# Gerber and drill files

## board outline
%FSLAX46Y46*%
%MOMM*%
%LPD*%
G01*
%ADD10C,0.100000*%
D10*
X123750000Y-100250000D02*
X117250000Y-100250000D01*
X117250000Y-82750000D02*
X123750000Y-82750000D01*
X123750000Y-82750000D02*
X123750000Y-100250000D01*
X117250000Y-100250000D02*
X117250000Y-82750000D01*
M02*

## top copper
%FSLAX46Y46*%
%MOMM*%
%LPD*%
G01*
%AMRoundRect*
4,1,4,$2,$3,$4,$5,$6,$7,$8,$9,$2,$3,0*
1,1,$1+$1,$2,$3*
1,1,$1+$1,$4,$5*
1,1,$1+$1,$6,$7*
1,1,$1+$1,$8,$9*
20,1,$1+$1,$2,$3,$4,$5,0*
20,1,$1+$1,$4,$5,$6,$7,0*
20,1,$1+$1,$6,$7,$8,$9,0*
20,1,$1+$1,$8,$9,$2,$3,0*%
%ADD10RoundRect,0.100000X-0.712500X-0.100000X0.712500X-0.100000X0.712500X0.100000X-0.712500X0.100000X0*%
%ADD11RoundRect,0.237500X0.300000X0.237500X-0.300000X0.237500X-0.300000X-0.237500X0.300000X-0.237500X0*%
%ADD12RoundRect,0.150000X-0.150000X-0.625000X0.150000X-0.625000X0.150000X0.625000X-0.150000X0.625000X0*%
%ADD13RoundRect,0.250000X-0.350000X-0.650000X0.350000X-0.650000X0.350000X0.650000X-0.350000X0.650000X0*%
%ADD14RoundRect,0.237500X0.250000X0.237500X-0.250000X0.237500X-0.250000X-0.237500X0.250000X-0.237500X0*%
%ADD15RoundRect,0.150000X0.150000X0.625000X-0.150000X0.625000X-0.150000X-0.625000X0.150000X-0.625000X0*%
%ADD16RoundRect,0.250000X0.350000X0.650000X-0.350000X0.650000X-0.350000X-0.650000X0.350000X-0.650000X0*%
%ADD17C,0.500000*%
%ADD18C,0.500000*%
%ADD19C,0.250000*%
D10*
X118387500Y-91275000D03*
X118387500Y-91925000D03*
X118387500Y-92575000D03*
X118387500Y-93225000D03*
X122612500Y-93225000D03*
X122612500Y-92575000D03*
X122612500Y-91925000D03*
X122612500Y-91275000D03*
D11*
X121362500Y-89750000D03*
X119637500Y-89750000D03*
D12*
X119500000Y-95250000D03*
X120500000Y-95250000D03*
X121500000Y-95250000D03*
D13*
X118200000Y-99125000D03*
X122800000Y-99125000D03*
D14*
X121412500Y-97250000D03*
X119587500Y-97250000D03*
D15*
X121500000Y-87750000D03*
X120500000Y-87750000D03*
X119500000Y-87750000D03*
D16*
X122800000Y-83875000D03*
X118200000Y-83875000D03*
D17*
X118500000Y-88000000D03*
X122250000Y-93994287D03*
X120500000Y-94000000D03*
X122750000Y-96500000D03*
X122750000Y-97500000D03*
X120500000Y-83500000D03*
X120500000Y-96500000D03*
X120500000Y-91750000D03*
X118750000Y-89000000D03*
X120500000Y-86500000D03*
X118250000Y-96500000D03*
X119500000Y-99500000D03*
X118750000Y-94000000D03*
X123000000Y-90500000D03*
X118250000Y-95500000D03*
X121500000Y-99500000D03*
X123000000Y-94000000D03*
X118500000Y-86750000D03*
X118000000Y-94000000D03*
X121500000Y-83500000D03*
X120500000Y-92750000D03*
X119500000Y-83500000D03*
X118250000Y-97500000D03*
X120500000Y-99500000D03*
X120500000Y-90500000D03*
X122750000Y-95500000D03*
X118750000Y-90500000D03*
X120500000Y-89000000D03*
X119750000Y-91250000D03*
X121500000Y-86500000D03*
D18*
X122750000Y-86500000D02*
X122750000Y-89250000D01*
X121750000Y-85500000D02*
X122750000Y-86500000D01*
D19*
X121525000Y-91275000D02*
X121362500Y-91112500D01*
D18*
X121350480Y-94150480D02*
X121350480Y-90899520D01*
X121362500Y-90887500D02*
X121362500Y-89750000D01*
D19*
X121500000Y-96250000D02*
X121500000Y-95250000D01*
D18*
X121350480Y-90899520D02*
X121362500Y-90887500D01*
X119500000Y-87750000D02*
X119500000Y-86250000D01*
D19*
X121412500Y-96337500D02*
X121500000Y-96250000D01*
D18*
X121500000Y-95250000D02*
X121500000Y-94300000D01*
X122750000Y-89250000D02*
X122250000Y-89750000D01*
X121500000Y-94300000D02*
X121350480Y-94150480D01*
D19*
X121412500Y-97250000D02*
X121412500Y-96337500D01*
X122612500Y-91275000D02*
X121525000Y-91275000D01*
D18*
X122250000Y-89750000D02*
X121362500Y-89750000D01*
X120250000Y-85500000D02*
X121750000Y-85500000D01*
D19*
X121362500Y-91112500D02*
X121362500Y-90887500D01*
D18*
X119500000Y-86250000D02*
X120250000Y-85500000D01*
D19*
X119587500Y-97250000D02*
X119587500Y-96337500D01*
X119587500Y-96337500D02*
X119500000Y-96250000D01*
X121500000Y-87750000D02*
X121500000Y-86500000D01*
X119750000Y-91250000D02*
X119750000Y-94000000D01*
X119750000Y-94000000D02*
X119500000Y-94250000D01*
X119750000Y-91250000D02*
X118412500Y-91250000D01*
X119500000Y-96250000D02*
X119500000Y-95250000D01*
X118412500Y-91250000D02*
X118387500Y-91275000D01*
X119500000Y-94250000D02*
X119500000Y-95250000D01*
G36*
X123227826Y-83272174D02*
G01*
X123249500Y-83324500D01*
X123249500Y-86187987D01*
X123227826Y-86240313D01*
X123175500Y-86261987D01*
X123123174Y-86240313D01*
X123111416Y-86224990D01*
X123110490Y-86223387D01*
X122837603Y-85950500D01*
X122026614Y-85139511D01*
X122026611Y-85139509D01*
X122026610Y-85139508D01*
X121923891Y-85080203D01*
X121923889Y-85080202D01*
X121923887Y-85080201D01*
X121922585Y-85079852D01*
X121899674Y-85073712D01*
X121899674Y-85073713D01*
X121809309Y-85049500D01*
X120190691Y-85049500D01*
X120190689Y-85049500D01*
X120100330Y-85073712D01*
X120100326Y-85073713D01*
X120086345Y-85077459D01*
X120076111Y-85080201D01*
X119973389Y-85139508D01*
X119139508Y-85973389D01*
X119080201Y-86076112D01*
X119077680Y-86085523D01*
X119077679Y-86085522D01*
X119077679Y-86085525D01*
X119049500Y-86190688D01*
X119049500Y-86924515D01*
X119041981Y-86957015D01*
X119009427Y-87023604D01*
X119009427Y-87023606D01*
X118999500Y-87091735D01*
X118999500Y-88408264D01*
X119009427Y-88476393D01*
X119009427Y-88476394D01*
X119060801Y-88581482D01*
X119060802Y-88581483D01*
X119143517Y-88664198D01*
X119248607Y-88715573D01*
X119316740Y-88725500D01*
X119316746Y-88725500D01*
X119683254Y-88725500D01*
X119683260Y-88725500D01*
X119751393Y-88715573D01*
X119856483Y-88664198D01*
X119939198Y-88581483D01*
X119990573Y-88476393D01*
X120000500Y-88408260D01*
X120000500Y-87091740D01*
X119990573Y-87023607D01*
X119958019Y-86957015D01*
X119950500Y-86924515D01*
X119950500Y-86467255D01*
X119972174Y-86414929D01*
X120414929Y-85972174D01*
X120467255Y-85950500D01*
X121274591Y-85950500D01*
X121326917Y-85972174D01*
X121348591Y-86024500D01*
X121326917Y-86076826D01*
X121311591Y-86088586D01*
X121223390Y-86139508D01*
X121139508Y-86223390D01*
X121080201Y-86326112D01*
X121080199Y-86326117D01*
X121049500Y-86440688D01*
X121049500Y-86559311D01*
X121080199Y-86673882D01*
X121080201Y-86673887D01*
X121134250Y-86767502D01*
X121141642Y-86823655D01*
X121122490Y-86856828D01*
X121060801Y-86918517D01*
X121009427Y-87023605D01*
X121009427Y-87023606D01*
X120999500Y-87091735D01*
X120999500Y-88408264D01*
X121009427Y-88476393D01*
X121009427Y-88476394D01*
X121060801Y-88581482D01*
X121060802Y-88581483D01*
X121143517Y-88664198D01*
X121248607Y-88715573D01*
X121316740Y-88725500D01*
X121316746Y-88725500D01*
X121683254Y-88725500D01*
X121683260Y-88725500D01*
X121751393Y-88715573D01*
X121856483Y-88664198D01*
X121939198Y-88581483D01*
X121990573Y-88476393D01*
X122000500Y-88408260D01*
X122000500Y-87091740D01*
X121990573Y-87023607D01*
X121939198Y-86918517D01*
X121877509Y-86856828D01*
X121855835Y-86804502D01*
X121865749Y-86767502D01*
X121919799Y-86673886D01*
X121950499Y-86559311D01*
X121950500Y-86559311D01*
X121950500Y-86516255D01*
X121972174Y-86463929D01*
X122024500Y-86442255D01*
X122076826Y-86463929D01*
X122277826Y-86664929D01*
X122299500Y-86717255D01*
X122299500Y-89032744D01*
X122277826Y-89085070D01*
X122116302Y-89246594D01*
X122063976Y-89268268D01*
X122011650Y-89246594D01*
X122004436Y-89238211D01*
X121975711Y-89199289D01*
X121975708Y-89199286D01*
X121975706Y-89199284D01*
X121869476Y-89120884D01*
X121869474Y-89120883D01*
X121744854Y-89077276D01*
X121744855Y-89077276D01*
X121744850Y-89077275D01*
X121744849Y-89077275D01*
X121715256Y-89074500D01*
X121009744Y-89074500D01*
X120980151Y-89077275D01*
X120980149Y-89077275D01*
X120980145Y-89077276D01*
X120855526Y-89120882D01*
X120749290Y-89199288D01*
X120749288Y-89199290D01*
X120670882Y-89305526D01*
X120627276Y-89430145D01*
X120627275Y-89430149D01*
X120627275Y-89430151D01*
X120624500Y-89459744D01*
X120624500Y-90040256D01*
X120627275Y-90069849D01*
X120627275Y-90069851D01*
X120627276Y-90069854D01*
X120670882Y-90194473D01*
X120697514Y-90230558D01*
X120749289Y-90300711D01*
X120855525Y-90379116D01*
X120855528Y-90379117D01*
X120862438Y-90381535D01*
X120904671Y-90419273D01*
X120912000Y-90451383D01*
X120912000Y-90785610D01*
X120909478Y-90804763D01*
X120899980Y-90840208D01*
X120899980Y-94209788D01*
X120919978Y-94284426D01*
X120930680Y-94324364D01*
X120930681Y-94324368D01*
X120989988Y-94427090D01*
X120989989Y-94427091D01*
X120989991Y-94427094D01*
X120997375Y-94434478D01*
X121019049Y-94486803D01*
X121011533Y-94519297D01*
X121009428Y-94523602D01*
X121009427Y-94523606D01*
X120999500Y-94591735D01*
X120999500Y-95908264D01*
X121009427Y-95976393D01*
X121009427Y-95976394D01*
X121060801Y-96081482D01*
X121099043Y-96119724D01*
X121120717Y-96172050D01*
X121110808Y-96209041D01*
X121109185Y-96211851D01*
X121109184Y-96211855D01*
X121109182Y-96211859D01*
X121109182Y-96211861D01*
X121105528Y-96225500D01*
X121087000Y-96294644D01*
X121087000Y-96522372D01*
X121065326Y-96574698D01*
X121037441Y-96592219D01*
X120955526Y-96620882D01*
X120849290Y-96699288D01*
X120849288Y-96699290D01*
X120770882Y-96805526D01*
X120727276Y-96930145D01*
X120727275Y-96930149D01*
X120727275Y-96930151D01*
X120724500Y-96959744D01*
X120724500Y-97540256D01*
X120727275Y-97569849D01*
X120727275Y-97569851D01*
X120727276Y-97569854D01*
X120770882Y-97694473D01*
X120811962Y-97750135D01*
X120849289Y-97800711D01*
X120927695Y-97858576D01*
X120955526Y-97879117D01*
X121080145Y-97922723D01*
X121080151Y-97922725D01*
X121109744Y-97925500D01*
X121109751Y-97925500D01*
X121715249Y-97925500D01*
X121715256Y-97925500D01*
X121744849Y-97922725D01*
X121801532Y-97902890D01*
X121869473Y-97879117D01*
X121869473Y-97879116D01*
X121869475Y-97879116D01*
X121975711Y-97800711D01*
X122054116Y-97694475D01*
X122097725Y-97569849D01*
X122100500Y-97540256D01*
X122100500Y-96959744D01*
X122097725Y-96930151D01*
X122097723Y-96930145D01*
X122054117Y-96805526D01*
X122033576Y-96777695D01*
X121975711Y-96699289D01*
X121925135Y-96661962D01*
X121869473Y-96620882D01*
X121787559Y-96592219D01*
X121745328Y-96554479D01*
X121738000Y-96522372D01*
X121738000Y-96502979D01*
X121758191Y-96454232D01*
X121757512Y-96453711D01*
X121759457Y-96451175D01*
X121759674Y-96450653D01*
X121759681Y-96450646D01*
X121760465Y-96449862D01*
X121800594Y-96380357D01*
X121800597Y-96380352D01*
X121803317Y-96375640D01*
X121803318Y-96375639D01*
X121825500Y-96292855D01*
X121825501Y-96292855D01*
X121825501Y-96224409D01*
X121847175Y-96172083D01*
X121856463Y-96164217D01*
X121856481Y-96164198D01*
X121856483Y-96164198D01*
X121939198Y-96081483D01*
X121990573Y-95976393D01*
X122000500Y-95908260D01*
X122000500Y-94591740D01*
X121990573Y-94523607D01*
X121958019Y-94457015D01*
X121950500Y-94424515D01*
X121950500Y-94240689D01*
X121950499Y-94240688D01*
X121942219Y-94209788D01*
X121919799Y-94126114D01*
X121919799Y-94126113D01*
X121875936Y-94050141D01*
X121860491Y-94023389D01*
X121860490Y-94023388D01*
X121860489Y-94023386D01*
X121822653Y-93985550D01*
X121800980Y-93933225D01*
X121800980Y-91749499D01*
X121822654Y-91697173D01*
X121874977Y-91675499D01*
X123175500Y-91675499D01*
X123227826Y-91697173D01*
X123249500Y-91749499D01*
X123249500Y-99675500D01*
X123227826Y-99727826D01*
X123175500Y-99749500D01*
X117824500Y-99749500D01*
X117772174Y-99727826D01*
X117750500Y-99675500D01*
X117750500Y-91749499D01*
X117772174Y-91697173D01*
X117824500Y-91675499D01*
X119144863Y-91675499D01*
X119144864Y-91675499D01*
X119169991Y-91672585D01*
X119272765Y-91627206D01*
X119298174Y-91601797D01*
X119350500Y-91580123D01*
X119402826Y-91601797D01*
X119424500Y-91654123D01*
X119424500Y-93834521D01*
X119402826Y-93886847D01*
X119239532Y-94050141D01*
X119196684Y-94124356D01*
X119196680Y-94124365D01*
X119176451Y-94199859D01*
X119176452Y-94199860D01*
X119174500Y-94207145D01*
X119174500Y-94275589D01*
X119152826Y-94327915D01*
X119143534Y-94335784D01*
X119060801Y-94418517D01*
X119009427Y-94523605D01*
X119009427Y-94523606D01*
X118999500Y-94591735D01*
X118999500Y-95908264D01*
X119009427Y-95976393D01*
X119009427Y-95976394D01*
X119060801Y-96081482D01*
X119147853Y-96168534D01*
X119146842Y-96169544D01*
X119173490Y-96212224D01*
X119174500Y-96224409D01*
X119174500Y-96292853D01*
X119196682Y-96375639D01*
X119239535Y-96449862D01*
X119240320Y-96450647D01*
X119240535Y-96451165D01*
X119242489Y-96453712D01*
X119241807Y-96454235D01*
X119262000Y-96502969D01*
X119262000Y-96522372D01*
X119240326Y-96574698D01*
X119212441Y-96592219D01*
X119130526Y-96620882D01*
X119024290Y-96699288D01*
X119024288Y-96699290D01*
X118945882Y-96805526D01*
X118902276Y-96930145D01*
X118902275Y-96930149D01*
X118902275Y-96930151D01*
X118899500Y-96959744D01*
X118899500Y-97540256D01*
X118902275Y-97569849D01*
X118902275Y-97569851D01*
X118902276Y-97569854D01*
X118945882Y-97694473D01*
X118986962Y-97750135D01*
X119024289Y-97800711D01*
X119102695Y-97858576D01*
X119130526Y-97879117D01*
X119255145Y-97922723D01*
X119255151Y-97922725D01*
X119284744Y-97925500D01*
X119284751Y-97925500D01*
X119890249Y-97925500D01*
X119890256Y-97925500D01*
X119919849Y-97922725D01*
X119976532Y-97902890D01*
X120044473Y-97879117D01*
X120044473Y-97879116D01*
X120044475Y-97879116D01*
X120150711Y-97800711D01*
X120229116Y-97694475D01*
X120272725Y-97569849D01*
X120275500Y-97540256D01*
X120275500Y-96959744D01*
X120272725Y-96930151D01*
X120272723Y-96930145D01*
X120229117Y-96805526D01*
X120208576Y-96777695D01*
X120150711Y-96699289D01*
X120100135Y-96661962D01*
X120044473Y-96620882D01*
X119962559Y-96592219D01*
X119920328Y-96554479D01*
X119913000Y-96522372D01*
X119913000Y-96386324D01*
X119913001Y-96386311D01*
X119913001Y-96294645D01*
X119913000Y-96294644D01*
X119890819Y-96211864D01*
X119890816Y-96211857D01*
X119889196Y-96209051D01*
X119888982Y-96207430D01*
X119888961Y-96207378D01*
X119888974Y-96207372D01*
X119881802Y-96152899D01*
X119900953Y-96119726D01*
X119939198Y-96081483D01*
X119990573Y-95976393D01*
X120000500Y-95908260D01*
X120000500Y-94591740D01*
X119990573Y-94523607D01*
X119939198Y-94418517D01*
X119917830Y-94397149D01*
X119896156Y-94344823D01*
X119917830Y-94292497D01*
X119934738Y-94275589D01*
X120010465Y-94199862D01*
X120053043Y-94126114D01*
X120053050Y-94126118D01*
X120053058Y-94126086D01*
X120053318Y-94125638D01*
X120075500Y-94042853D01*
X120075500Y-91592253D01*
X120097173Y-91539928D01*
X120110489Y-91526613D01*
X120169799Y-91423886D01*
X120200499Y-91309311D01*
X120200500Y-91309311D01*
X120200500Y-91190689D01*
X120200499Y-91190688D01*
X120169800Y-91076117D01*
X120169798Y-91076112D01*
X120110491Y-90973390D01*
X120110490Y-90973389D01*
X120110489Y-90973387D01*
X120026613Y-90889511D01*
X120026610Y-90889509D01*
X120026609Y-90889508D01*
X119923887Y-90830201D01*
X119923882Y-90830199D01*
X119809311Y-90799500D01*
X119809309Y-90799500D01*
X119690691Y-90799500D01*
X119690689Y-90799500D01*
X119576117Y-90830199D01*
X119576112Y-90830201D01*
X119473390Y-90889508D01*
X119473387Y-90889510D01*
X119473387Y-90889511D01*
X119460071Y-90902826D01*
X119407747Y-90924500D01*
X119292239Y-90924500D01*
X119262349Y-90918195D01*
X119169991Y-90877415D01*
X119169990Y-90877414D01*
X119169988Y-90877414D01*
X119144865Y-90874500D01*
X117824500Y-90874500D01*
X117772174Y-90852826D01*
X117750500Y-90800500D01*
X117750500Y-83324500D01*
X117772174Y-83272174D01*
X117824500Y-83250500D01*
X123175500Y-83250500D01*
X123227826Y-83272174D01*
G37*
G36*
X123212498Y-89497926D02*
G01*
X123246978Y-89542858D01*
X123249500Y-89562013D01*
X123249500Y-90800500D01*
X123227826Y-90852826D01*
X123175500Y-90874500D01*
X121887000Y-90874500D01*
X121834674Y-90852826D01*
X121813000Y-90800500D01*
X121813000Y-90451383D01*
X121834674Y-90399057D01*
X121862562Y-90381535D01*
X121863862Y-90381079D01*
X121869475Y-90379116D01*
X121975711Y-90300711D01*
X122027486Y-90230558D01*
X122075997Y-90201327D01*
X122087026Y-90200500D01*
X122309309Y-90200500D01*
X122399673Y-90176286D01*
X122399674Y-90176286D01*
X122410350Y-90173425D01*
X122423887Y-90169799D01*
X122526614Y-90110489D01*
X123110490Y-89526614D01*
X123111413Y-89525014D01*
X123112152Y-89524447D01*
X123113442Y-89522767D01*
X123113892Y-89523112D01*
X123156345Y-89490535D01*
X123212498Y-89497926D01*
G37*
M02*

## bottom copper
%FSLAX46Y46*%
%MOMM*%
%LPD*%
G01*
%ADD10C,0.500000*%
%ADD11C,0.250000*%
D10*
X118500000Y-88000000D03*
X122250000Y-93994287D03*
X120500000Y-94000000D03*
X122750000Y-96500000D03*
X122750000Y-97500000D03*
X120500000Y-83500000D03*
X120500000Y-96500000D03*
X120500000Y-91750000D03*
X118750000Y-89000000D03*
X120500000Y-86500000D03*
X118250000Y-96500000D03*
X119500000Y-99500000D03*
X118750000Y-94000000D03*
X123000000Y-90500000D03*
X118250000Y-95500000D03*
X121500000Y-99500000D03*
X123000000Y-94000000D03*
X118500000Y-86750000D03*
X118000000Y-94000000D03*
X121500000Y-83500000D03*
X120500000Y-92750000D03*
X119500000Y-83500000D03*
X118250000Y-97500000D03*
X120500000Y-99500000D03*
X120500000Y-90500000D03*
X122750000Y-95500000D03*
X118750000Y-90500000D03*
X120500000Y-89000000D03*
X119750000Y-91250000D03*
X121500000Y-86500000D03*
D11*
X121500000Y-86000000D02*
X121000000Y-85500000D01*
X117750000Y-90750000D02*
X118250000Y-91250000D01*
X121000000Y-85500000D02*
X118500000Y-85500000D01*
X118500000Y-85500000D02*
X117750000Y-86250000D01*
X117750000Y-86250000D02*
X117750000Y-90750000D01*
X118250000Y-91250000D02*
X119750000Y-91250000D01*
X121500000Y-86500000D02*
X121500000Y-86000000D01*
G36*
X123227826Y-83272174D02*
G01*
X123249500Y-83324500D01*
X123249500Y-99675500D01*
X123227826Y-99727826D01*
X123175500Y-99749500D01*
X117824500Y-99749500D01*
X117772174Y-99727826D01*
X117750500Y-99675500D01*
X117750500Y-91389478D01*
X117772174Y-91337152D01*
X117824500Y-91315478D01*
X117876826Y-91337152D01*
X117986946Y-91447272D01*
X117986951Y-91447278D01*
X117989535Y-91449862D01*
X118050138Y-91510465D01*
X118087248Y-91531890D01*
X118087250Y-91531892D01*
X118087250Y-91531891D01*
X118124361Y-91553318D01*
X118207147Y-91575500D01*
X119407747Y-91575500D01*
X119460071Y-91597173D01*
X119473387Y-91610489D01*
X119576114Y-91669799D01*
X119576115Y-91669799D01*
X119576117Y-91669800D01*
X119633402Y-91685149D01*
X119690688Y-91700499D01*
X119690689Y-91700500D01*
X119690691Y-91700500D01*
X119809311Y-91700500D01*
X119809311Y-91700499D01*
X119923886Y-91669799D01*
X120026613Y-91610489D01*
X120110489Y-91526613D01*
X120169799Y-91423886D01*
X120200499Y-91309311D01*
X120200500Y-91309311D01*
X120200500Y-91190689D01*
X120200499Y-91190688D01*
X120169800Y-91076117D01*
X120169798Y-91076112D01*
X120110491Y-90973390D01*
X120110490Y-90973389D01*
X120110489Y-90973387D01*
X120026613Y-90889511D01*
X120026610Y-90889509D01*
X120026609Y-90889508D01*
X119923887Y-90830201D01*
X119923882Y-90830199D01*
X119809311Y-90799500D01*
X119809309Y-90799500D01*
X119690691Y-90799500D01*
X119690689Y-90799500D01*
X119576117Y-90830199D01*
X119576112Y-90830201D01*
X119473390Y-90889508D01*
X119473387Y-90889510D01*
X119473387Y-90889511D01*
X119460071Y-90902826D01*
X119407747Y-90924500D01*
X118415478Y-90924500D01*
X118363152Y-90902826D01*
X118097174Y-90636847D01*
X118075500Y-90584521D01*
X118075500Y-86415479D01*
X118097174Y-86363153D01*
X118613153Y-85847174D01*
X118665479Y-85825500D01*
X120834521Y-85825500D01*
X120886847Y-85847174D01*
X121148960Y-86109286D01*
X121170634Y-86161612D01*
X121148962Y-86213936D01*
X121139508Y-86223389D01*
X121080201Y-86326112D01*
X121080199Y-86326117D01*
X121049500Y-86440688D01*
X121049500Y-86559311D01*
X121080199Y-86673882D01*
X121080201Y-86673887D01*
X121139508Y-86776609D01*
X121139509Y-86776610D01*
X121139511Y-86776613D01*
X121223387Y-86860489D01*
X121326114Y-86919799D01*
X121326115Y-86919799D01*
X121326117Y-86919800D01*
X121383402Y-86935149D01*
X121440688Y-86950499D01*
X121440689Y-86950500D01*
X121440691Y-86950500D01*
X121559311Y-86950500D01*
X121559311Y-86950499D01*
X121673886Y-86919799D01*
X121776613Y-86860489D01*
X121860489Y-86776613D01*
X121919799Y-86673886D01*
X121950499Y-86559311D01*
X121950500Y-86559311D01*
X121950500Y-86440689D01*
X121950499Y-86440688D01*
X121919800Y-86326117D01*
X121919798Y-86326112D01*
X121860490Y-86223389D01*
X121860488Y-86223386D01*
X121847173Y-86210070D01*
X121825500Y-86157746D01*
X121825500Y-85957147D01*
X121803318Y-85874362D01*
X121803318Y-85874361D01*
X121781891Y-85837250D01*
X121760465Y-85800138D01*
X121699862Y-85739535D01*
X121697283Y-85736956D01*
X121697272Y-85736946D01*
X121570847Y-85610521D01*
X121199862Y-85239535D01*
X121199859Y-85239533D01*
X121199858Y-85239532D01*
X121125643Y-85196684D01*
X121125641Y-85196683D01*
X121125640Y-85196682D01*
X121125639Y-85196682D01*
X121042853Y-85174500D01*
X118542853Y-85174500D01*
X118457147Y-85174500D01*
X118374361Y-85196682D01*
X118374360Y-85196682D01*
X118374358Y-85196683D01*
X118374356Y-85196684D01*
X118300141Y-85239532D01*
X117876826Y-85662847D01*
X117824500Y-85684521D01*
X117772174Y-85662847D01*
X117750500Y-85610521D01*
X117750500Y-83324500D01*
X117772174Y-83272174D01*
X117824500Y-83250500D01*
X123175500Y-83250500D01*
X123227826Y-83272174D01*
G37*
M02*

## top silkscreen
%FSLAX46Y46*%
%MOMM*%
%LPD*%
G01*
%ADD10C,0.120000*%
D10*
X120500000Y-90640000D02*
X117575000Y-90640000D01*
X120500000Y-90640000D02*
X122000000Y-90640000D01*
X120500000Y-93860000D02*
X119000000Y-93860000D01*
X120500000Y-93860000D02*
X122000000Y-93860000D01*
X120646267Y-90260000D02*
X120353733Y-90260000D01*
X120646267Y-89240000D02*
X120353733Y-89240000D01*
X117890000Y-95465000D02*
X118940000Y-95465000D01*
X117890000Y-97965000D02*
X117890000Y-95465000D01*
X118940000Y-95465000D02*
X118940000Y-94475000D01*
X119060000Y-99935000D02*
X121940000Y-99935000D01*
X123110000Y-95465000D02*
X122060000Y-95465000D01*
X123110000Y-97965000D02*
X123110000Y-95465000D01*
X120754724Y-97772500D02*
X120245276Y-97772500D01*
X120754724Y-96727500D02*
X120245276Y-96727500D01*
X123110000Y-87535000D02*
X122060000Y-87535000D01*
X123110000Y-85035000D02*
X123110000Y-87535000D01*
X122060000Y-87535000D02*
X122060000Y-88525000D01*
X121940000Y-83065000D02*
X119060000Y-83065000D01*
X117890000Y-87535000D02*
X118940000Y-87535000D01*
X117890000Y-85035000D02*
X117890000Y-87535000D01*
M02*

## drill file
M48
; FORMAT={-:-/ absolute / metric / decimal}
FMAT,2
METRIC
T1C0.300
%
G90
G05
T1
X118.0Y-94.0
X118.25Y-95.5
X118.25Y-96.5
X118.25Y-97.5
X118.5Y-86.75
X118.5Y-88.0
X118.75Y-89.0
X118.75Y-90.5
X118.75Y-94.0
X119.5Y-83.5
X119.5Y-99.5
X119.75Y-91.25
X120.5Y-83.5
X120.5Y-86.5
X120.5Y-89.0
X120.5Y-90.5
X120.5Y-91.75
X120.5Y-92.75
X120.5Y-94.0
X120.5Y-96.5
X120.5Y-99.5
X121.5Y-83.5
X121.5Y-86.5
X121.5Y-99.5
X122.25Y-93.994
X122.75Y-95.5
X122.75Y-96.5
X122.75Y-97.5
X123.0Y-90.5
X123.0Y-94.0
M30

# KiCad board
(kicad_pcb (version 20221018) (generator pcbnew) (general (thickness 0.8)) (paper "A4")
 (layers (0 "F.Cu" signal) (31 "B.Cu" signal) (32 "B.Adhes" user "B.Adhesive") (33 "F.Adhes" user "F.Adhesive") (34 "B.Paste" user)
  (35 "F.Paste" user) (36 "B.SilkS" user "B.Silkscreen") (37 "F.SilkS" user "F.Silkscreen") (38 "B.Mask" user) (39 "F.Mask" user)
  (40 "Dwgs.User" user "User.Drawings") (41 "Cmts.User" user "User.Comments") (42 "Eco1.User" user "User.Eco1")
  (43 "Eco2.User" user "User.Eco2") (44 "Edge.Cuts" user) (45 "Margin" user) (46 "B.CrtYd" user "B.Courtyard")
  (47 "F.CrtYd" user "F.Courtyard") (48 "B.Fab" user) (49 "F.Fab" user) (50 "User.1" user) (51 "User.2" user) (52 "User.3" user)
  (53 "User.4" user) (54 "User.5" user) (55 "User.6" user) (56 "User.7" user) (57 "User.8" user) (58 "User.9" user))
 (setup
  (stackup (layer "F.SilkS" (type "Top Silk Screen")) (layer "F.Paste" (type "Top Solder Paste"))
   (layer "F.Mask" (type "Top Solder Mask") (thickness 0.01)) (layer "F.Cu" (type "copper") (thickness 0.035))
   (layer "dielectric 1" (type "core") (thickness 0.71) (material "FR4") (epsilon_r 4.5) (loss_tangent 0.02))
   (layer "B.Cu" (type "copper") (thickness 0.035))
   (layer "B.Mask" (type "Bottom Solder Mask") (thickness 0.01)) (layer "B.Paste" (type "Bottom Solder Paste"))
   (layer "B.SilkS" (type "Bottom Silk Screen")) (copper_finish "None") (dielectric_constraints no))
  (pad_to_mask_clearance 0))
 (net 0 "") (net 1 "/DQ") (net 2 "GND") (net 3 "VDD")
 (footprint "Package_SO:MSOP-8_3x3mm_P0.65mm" (layer "F.Cu") (at 120.5 92.25)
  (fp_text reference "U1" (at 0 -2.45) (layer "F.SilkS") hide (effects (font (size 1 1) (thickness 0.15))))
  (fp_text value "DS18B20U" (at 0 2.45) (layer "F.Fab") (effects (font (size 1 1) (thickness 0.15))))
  (fp_line (start 0 -1.61) (end -2.925 -1.61) (stroke (width 0.12) (type solid)) (layer "F.SilkS"))
  (fp_line (start 0 -1.61) (end 1.5 -1.61) (stroke (width 0.12) (type solid)) (layer "F.SilkS"))
  (fp_line (start 0 1.61) (end -1.5 1.61) (stroke (width 0.12) (type solid)) (layer "F.SilkS"))
  (fp_line (start 0 1.61) (end 1.5 1.61) (stroke (width 0.12) (type solid)) (layer "F.SilkS"))
  (pad "1" smd roundrect (at -2.1125 -0.975) (size 1.625 0.4) (layers "F.Cu" "F.Paste" "F.Mask") (roundrect_rratio 0.25) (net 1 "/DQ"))
  (pad "2" smd roundrect (at -2.1125 -0.325) (size 1.625 0.4) (layers "F.Cu" "F.Paste" "F.Mask") (roundrect_rratio 0.25) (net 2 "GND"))
  (pad "3" smd roundrect (at -2.1125 0.325) (size 1.625 0.4) (layers "F.Cu" "F.Paste" "F.Mask") (roundrect_rratio 0.25) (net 2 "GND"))
  (pad "4" smd roundrect (at -2.1125 0.975) (size 1.625 0.4) (layers "F.Cu" "F.Paste" "F.Mask") (roundrect_rratio 0.25) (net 2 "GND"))
  (pad "5" smd roundrect (at 2.1125 0.975) (size 1.625 0.4) (layers "F.Cu" "F.Paste" "F.Mask") (roundrect_rratio 0.25) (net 2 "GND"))
  (pad "6" smd roundrect (at 2.1125 0.325) (size 1.625 0.4) (layers "F.Cu" "F.Paste" "F.Mask") (roundrect_rratio 0.25) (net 2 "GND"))
  (pad "7" smd roundrect (at 2.1125 -0.325) (size 1.625 0.4) (layers "F.Cu" "F.Paste" "F.Mask") (roundrect_rratio 0.25) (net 2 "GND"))
  (pad "8" smd roundrect (at 2.1125 -0.975) (size 1.625 0.4) (layers "F.Cu" "F.Paste" "F.Mask") (roundrect_rratio 0.25) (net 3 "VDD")))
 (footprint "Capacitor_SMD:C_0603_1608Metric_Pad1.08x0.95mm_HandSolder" (layer "F.Cu") (at 120.5 89.75 180)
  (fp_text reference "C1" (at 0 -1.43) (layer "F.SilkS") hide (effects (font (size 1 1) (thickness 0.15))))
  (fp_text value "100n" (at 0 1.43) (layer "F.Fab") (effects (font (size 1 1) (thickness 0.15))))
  (fp_line (start -0.146267 -0.51) (end 0.146267 -0.51) (stroke (width 0.12) (type solid)) (layer "F.SilkS"))
  (fp_line (start -0.146267 0.51) (end 0.146267 0.51) (stroke (width 0.12) (type solid)) (layer "F.SilkS"))
  (pad "1" smd roundrect (at -0.8625 0 180) (size 1.075 0.95) (layers "F.Cu" "F.Paste" "F.Mask") (roundrect_rratio 0.25) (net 3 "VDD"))
  (pad "2" smd roundrect (at 0.8625 0 180) (size 1.075 0.95) (layers "F.Cu" "F.Paste" "F.Mask") (roundrect_rratio 0.25) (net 2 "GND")))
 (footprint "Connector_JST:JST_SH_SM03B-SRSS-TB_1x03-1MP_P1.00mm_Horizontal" (layer "F.Cu") (at 120.5 97.25)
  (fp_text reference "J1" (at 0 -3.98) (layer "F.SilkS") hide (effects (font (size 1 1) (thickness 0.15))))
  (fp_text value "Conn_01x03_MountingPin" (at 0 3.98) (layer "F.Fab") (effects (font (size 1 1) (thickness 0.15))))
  (fp_line (start -2.61 -1.785) (end -1.56 -1.785) (stroke (width 0.12) (type solid)) (layer "F.SilkS"))
  (fp_line (start -2.61 0.715) (end -2.61 -1.785) (stroke (width 0.12) (type solid)) (layer "F.SilkS"))
  (fp_line (start -1.56 -1.785) (end -1.56 -2.775) (stroke (width 0.12) (type solid)) (layer "F.SilkS"))
  (fp_line (start -1.44 2.685) (end 1.44 2.685) (stroke (width 0.12) (type solid)) (layer "F.SilkS"))
  (fp_line (start 2.61 -1.785) (end 1.56 -1.785) (stroke (width 0.12) (type solid)) (layer "F.SilkS"))
  (fp_line (start 2.61 0.715) (end 2.61 -1.785) (stroke (width 0.12) (type solid)) (layer "F.SilkS"))
  (pad "1" smd roundrect (at -1 -2) (size 0.6 1.55) (layers "F.Cu" "F.Paste" "F.Mask") (roundrect_rratio 0.25) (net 1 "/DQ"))
  (pad "2" smd roundrect (at 0 -2) (size 0.6 1.55) (layers "F.Cu" "F.Paste" "F.Mask") (roundrect_rratio 0.25) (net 2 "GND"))
  (pad "3" smd roundrect (at 1 -2) (size 0.6 1.55) (layers "F.Cu" "F.Paste" "F.Mask") (roundrect_rratio 0.25) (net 3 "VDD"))
  (pad "MP" smd roundrect (at -2.3 1.875) (size 1.2 1.8) (layers "F.Cu" "F.Paste" "F.Mask") (roundrect_rratio 0.2083333333) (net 2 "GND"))
  (pad "MP" smd roundrect (at 2.3 1.875) (size 1.2 1.8) (layers "F.Cu" "F.Paste" "F.Mask") (roundrect_rratio 0.2083333333) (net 2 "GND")))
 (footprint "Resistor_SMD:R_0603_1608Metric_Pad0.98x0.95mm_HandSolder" (layer "F.Cu") (at 120.5 97.25 180)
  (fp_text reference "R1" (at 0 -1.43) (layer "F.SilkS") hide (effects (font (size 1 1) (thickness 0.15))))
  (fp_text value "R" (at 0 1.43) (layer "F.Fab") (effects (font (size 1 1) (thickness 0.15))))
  (fp_line (start -0.254724 -0.5225) (end 0.254724 -0.5225) (stroke (width 0.12) (type solid)) (layer "F.SilkS"))
  (fp_line (start -0.254724 0.5225) (end 0.254724 0.5225) (stroke (width 0.12) (type solid)) (layer "F.SilkS"))
  (pad "1" smd roundrect (at -0.9125 0 180) (size 0.975 0.95) (layers "F.Cu" "F.Paste" "F.Mask") (roundrect_rratio 0.25) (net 3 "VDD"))
  (pad "2" smd roundrect (at 0.9125 0 180) (size 0.975 0.95) (layers "F.Cu" "F.Paste" "F.Mask") (roundrect_rratio 0.25) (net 1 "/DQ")))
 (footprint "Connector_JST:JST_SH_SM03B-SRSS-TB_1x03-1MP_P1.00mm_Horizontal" (layer "F.Cu") (at 120.5 85.75 180)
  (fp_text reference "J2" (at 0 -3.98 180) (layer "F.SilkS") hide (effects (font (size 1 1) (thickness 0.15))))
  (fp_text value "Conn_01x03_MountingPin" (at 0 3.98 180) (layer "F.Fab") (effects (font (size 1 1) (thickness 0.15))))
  (fp_line (start -2.61 -1.785) (end -1.56 -1.785) (stroke (width 0.12) (type solid)) (layer "F.SilkS"))
  (fp_line (start -2.61 0.715) (end -2.61 -1.785) (stroke (width 0.12) (type solid)) (layer "F.SilkS"))
  (fp_line (start -1.56 -1.785) (end -1.56 -2.775) (stroke (width 0.12) (type solid)) (layer "F.SilkS"))
  (fp_line (start -1.44 2.685) (end 1.44 2.685) (stroke (width 0.12) (type solid)) (layer "F.SilkS"))
  (fp_line (start 2.61 -1.785) (end 1.56 -1.785) (stroke (width 0.12) (type solid)) (layer "F.SilkS"))
  (fp_line (start 2.61 0.715) (end 2.61 -1.785) (stroke (width 0.12) (type solid)) (layer "F.SilkS"))
  (pad "1" smd roundrect (at -1 -2 180) (size 0.6 1.55) (layers "F.Cu" "F.Paste" "F.Mask") (roundrect_rratio 0.25) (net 1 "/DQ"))
  (pad "2" smd roundrect (at 0 -2 180) (size 0.6 1.55) (layers "F.Cu" "F.Paste" "F.Mask") (roundrect_rratio 0.25) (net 2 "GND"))
  (pad "3" smd roundrect (at 1 -2 180) (size 0.6 1.55) (layers "F.Cu" "F.Paste" "F.Mask") (roundrect_rratio 0.25) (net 3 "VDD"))
  (pad "MP" smd roundrect (at -2.3 1.875 180) (size 1.2 1.8) (layers "F.Cu" "F.Paste" "F.Mask") (roundrect_rratio 0.2083333333)
   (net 2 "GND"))
  (pad "MP" smd roundrect (at 2.3 1.875 180) (size 1.2 1.8) (layers "F.Cu" "F.Paste" "F.Mask") (roundrect_rratio 0.2083333333) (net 2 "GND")))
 (gr_line (start 123.75 100.25) (end 117.25 100.25) (stroke (width 0.1) (type solid)) (layer "Edge.Cuts"))
 (gr_line (start 117.25 82.75) (end 123.75 82.75) (stroke (width 0.1) (type solid)) (layer "Edge.Cuts"))
 (gr_line (start 123.75 82.75) (end 123.75 100.25) (stroke (width 0.1) (type solid)) (layer "Edge.Cuts"))
 (gr_line (start 117.25 100.25) (end 117.25 82.75) (stroke (width 0.1) (type solid)) (layer "Edge.Cuts"))
 (segment (start 122.75 86.5) (end 122.75 89.25) (width 0.5) (layer "F.Cu") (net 3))
 (segment (start 121.75 85.5) (end 122.75 86.5) (width 0.5) (layer "F.Cu") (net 3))
 (segment (start 121.525 91.275) (end 121.3625 91.1125) (width 0.25) (layer "F.Cu") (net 3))
 (segment (start 121.35048 94.15048) (end 121.35048 90.89952) (width 0.5) (layer "F.Cu") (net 3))
 (segment (start 121.3625 90.8875) (end 121.3625 89.75) (width 0.5) (layer "F.Cu") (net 3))
 (segment (start 121.5 96.25) (end 121.5 95.25) (width 0.25) (layer "F.Cu") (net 3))
 (segment (start 121.35048 90.89952) (end 121.3625 90.8875) (width 0.5) (layer "F.Cu") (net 3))
 (segment (start 119.5 87.75) (end 119.5 86.25) (width 0.5) (layer "F.Cu") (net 3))
 (segment (start 121.4125 96.3375) (end 121.5 96.25) (width 0.25) (layer "F.Cu") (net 3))
 (segment (start 121.5 95.25) (end 121.5 94.3) (width 0.5) (layer "F.Cu") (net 3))
 (segment (start 122.75 89.25) (end 122.25 89.75) (width 0.5) (layer "F.Cu") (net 3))
 (segment (start 121.5 94.3) (end 121.35048 94.15048) (width 0.5) (layer "F.Cu") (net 3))
 (segment (start 121.4125 97.25) (end 121.4125 96.3375) (width 0.25) (layer "F.Cu") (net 3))
 (segment (start 122.6125 91.275) (end 121.525 91.275) (width 0.25) (layer "F.Cu") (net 3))
 (segment (start 122.25 89.75) (end 121.3625 89.75) (width 0.5) (layer "F.Cu") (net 3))
 (segment (start 120.25 85.5) (end 121.75 85.5) (width 0.5) (layer "F.Cu") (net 3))
 (segment (start 121.3625 91.1125) (end 121.3625 90.8875) (width 0.25) (layer "F.Cu") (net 3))
 (segment (start 119.5 86.25) (end 120.25 85.5) (width 0.5) (layer "F.Cu") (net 3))
 (via (at 118.5 88) (size 0.5) (drill 0.3) (layers "F.Cu" "B.Cu") (free) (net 2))
 (via (at 122.25 93.994287) (size 0.5) (drill 0.3) (layers "F.Cu" "B.Cu") (free) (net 2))
 (via (at 120.5 94) (size 0.5) (drill 0.3) (layers "F.Cu" "B.Cu") (free) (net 2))
 (via (at 122.75 96.5) (size 0.5) (drill 0.3) (layers "F.Cu" "B.Cu") (free) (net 2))
 (via (at 122.75 97.5) (size 0.5) (drill 0.3) (layers "F.Cu" "B.Cu") (free) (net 2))
 (via (at 120.5 83.5) (size 0.5) (drill 0.3) (layers "F.Cu" "B.Cu") (free) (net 2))
 (via (at 120.5 96.5) (size 0.5) (drill 0.3) (layers "F.Cu" "B.Cu") (free) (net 2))
 (via (at 120.5 91.75) (size 0.5) (drill 0.3) (layers "F.Cu" "B.Cu") (free) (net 2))
 (via (at 118.75 89) (size 0.5) (drill 0.3) (layers "F.Cu" "B.Cu") (free) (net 2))
 (via (at 120.5 86.5) (size 0.5) (drill 0.3) (layers "F.Cu" "B.Cu") (free) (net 2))
 (via (at 118.25 96.5) (size 0.5) (drill 0.3) (layers "F.Cu" "B.Cu") (free) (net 2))
 (via (at 119.5 99.5) (size 0.5) (drill 0.3) (layers "F.Cu" "B.Cu") (free) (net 2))
 (via (at 118.75 94) (size 0.5) (drill 0.3) (layers "F.Cu" "B.Cu") (free) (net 2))
 (via (at 123 90.5) (size 0.5) (drill 0.3) (layers "F.Cu" "B.Cu") (free) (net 2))
 (via (at 118.25 95.5) (size 0.5) (drill 0.3) (layers "F.Cu" "B.Cu") (free) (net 2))
 (via (at 121.5 99.5) (size 0.5) (drill 0.3) (layers "F.Cu" "B.Cu") (free) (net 2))
 (via (at 123 94) (size 0.5) (drill 0.3) (layers "F.Cu" "B.Cu") (free) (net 2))
 (via (at 118.5 86.75) (size 0.5) (drill 0.3) (layers "F.Cu" "B.Cu") (free) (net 2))
 (via (at 118 94) (size 0.5) (drill 0.3) (layers "F.Cu" "B.Cu") (free) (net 2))
 (via (at 121.5 83.5) (size 0.5) (drill 0.3) (layers "F.Cu" "B.Cu") (free) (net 2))
 (via (at 120.5 92.75) (size 0.5) (drill 0.3) (layers "F.Cu" "B.Cu") (free) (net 2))
 (via (at 119.5 83.5) (size 0.5) (drill 0.3) (layers "F.Cu" "B.Cu") (free) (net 2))
 (via (at 118.25 97.5) (size 0.5) (drill 0.3) (layers "F.Cu" "B.Cu") (free) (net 2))
 (via (at 120.5 99.5) (size 0.5) (drill 0.3) (layers "F.Cu" "B.Cu") (free) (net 2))
 (via (at 120.5 90.5) (size 0.5) (drill 0.3) (layers "F.Cu" "B.Cu") (free) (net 2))
 (via (at 122.75 95.5) (size 0.5) (drill 0.3) (layers "F.Cu" "B.Cu") (free) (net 2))
 (via (at 118.75 90.5) (size 0.5) (drill 0.3) (layers "F.Cu" "B.Cu") (free) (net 2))
 (via (at 120.5 89) (size 0.5) (drill 0.3) (layers "F.Cu" "B.Cu") (free) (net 2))
 (segment (start 119.5875 97.25) (end 119.5875 96.3375) (width 0.25) (layer "F.Cu") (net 1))
 (segment (start 119.5875 96.3375) (end 119.5 96.25) (width 0.25) (layer "F.Cu") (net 1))
 (segment (start 121.5 87.75) (end 121.5 86.5) (width 0.25) (layer "F.Cu") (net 1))
 (segment (start 119.75 91.25) (end 119.75 94) (width 0.25) (layer "F.Cu") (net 1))
 (segment (start 119.75 94) (end 119.5 94.25) (width 0.25) (layer "F.Cu") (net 1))
 (segment (start 119.75 91.25) (end 118.4125 91.25) (width 0.25) (layer "F.Cu") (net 1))
 (segment (start 119.5 96.25) (end 119.5 95.25) (width 0.25) (layer "F.Cu") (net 1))
 (segment (start 118.4125 91.25) (end 118.3875 91.275) (width 0.25) (layer "F.Cu") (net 1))
 (segment (start 119.5 94.25) (end 119.5 95.25) (width 0.25) (layer "F.Cu") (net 1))
 (via (at 119.75 91.25) (size 0.5) (drill 0.3) (layers "F.Cu" "B.Cu") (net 1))
 (via (at 121.5 86.5) (size 0.5) (drill 0.3) (layers "F.Cu" "B.Cu") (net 1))
 (segment (start 121.5 86) (end 121 85.5) (width 0.25) (layer "B.Cu") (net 1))
 (segment (start 117.75 90.75) (end 118.25 91.25) (width 0.25) (layer "B.Cu") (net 1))
 (segment (start 121 85.5) (end 118.5 85.5) (width 0.25) (layer "B.Cu") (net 1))
 (segment (start 118.5 85.5) (end 117.75 86.25) (width 0.25) (layer "B.Cu") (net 1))
 (segment (start 117.75 86.25) (end 117.75 90.75) (width 0.25) (layer "B.Cu") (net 1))
 (segment (start 118.25 91.25) (end 119.75 91.25) (width 0.25) (layer "B.Cu") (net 1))
 (segment (start 121.5 86.5) (end 121.5 86) (width 0.25) (layer "B.Cu") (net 1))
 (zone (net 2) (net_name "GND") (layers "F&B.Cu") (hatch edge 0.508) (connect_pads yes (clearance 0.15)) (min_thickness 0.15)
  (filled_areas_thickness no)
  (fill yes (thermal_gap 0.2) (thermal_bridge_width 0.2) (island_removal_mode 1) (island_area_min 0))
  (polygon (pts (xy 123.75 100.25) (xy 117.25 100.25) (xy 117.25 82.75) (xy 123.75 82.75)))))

